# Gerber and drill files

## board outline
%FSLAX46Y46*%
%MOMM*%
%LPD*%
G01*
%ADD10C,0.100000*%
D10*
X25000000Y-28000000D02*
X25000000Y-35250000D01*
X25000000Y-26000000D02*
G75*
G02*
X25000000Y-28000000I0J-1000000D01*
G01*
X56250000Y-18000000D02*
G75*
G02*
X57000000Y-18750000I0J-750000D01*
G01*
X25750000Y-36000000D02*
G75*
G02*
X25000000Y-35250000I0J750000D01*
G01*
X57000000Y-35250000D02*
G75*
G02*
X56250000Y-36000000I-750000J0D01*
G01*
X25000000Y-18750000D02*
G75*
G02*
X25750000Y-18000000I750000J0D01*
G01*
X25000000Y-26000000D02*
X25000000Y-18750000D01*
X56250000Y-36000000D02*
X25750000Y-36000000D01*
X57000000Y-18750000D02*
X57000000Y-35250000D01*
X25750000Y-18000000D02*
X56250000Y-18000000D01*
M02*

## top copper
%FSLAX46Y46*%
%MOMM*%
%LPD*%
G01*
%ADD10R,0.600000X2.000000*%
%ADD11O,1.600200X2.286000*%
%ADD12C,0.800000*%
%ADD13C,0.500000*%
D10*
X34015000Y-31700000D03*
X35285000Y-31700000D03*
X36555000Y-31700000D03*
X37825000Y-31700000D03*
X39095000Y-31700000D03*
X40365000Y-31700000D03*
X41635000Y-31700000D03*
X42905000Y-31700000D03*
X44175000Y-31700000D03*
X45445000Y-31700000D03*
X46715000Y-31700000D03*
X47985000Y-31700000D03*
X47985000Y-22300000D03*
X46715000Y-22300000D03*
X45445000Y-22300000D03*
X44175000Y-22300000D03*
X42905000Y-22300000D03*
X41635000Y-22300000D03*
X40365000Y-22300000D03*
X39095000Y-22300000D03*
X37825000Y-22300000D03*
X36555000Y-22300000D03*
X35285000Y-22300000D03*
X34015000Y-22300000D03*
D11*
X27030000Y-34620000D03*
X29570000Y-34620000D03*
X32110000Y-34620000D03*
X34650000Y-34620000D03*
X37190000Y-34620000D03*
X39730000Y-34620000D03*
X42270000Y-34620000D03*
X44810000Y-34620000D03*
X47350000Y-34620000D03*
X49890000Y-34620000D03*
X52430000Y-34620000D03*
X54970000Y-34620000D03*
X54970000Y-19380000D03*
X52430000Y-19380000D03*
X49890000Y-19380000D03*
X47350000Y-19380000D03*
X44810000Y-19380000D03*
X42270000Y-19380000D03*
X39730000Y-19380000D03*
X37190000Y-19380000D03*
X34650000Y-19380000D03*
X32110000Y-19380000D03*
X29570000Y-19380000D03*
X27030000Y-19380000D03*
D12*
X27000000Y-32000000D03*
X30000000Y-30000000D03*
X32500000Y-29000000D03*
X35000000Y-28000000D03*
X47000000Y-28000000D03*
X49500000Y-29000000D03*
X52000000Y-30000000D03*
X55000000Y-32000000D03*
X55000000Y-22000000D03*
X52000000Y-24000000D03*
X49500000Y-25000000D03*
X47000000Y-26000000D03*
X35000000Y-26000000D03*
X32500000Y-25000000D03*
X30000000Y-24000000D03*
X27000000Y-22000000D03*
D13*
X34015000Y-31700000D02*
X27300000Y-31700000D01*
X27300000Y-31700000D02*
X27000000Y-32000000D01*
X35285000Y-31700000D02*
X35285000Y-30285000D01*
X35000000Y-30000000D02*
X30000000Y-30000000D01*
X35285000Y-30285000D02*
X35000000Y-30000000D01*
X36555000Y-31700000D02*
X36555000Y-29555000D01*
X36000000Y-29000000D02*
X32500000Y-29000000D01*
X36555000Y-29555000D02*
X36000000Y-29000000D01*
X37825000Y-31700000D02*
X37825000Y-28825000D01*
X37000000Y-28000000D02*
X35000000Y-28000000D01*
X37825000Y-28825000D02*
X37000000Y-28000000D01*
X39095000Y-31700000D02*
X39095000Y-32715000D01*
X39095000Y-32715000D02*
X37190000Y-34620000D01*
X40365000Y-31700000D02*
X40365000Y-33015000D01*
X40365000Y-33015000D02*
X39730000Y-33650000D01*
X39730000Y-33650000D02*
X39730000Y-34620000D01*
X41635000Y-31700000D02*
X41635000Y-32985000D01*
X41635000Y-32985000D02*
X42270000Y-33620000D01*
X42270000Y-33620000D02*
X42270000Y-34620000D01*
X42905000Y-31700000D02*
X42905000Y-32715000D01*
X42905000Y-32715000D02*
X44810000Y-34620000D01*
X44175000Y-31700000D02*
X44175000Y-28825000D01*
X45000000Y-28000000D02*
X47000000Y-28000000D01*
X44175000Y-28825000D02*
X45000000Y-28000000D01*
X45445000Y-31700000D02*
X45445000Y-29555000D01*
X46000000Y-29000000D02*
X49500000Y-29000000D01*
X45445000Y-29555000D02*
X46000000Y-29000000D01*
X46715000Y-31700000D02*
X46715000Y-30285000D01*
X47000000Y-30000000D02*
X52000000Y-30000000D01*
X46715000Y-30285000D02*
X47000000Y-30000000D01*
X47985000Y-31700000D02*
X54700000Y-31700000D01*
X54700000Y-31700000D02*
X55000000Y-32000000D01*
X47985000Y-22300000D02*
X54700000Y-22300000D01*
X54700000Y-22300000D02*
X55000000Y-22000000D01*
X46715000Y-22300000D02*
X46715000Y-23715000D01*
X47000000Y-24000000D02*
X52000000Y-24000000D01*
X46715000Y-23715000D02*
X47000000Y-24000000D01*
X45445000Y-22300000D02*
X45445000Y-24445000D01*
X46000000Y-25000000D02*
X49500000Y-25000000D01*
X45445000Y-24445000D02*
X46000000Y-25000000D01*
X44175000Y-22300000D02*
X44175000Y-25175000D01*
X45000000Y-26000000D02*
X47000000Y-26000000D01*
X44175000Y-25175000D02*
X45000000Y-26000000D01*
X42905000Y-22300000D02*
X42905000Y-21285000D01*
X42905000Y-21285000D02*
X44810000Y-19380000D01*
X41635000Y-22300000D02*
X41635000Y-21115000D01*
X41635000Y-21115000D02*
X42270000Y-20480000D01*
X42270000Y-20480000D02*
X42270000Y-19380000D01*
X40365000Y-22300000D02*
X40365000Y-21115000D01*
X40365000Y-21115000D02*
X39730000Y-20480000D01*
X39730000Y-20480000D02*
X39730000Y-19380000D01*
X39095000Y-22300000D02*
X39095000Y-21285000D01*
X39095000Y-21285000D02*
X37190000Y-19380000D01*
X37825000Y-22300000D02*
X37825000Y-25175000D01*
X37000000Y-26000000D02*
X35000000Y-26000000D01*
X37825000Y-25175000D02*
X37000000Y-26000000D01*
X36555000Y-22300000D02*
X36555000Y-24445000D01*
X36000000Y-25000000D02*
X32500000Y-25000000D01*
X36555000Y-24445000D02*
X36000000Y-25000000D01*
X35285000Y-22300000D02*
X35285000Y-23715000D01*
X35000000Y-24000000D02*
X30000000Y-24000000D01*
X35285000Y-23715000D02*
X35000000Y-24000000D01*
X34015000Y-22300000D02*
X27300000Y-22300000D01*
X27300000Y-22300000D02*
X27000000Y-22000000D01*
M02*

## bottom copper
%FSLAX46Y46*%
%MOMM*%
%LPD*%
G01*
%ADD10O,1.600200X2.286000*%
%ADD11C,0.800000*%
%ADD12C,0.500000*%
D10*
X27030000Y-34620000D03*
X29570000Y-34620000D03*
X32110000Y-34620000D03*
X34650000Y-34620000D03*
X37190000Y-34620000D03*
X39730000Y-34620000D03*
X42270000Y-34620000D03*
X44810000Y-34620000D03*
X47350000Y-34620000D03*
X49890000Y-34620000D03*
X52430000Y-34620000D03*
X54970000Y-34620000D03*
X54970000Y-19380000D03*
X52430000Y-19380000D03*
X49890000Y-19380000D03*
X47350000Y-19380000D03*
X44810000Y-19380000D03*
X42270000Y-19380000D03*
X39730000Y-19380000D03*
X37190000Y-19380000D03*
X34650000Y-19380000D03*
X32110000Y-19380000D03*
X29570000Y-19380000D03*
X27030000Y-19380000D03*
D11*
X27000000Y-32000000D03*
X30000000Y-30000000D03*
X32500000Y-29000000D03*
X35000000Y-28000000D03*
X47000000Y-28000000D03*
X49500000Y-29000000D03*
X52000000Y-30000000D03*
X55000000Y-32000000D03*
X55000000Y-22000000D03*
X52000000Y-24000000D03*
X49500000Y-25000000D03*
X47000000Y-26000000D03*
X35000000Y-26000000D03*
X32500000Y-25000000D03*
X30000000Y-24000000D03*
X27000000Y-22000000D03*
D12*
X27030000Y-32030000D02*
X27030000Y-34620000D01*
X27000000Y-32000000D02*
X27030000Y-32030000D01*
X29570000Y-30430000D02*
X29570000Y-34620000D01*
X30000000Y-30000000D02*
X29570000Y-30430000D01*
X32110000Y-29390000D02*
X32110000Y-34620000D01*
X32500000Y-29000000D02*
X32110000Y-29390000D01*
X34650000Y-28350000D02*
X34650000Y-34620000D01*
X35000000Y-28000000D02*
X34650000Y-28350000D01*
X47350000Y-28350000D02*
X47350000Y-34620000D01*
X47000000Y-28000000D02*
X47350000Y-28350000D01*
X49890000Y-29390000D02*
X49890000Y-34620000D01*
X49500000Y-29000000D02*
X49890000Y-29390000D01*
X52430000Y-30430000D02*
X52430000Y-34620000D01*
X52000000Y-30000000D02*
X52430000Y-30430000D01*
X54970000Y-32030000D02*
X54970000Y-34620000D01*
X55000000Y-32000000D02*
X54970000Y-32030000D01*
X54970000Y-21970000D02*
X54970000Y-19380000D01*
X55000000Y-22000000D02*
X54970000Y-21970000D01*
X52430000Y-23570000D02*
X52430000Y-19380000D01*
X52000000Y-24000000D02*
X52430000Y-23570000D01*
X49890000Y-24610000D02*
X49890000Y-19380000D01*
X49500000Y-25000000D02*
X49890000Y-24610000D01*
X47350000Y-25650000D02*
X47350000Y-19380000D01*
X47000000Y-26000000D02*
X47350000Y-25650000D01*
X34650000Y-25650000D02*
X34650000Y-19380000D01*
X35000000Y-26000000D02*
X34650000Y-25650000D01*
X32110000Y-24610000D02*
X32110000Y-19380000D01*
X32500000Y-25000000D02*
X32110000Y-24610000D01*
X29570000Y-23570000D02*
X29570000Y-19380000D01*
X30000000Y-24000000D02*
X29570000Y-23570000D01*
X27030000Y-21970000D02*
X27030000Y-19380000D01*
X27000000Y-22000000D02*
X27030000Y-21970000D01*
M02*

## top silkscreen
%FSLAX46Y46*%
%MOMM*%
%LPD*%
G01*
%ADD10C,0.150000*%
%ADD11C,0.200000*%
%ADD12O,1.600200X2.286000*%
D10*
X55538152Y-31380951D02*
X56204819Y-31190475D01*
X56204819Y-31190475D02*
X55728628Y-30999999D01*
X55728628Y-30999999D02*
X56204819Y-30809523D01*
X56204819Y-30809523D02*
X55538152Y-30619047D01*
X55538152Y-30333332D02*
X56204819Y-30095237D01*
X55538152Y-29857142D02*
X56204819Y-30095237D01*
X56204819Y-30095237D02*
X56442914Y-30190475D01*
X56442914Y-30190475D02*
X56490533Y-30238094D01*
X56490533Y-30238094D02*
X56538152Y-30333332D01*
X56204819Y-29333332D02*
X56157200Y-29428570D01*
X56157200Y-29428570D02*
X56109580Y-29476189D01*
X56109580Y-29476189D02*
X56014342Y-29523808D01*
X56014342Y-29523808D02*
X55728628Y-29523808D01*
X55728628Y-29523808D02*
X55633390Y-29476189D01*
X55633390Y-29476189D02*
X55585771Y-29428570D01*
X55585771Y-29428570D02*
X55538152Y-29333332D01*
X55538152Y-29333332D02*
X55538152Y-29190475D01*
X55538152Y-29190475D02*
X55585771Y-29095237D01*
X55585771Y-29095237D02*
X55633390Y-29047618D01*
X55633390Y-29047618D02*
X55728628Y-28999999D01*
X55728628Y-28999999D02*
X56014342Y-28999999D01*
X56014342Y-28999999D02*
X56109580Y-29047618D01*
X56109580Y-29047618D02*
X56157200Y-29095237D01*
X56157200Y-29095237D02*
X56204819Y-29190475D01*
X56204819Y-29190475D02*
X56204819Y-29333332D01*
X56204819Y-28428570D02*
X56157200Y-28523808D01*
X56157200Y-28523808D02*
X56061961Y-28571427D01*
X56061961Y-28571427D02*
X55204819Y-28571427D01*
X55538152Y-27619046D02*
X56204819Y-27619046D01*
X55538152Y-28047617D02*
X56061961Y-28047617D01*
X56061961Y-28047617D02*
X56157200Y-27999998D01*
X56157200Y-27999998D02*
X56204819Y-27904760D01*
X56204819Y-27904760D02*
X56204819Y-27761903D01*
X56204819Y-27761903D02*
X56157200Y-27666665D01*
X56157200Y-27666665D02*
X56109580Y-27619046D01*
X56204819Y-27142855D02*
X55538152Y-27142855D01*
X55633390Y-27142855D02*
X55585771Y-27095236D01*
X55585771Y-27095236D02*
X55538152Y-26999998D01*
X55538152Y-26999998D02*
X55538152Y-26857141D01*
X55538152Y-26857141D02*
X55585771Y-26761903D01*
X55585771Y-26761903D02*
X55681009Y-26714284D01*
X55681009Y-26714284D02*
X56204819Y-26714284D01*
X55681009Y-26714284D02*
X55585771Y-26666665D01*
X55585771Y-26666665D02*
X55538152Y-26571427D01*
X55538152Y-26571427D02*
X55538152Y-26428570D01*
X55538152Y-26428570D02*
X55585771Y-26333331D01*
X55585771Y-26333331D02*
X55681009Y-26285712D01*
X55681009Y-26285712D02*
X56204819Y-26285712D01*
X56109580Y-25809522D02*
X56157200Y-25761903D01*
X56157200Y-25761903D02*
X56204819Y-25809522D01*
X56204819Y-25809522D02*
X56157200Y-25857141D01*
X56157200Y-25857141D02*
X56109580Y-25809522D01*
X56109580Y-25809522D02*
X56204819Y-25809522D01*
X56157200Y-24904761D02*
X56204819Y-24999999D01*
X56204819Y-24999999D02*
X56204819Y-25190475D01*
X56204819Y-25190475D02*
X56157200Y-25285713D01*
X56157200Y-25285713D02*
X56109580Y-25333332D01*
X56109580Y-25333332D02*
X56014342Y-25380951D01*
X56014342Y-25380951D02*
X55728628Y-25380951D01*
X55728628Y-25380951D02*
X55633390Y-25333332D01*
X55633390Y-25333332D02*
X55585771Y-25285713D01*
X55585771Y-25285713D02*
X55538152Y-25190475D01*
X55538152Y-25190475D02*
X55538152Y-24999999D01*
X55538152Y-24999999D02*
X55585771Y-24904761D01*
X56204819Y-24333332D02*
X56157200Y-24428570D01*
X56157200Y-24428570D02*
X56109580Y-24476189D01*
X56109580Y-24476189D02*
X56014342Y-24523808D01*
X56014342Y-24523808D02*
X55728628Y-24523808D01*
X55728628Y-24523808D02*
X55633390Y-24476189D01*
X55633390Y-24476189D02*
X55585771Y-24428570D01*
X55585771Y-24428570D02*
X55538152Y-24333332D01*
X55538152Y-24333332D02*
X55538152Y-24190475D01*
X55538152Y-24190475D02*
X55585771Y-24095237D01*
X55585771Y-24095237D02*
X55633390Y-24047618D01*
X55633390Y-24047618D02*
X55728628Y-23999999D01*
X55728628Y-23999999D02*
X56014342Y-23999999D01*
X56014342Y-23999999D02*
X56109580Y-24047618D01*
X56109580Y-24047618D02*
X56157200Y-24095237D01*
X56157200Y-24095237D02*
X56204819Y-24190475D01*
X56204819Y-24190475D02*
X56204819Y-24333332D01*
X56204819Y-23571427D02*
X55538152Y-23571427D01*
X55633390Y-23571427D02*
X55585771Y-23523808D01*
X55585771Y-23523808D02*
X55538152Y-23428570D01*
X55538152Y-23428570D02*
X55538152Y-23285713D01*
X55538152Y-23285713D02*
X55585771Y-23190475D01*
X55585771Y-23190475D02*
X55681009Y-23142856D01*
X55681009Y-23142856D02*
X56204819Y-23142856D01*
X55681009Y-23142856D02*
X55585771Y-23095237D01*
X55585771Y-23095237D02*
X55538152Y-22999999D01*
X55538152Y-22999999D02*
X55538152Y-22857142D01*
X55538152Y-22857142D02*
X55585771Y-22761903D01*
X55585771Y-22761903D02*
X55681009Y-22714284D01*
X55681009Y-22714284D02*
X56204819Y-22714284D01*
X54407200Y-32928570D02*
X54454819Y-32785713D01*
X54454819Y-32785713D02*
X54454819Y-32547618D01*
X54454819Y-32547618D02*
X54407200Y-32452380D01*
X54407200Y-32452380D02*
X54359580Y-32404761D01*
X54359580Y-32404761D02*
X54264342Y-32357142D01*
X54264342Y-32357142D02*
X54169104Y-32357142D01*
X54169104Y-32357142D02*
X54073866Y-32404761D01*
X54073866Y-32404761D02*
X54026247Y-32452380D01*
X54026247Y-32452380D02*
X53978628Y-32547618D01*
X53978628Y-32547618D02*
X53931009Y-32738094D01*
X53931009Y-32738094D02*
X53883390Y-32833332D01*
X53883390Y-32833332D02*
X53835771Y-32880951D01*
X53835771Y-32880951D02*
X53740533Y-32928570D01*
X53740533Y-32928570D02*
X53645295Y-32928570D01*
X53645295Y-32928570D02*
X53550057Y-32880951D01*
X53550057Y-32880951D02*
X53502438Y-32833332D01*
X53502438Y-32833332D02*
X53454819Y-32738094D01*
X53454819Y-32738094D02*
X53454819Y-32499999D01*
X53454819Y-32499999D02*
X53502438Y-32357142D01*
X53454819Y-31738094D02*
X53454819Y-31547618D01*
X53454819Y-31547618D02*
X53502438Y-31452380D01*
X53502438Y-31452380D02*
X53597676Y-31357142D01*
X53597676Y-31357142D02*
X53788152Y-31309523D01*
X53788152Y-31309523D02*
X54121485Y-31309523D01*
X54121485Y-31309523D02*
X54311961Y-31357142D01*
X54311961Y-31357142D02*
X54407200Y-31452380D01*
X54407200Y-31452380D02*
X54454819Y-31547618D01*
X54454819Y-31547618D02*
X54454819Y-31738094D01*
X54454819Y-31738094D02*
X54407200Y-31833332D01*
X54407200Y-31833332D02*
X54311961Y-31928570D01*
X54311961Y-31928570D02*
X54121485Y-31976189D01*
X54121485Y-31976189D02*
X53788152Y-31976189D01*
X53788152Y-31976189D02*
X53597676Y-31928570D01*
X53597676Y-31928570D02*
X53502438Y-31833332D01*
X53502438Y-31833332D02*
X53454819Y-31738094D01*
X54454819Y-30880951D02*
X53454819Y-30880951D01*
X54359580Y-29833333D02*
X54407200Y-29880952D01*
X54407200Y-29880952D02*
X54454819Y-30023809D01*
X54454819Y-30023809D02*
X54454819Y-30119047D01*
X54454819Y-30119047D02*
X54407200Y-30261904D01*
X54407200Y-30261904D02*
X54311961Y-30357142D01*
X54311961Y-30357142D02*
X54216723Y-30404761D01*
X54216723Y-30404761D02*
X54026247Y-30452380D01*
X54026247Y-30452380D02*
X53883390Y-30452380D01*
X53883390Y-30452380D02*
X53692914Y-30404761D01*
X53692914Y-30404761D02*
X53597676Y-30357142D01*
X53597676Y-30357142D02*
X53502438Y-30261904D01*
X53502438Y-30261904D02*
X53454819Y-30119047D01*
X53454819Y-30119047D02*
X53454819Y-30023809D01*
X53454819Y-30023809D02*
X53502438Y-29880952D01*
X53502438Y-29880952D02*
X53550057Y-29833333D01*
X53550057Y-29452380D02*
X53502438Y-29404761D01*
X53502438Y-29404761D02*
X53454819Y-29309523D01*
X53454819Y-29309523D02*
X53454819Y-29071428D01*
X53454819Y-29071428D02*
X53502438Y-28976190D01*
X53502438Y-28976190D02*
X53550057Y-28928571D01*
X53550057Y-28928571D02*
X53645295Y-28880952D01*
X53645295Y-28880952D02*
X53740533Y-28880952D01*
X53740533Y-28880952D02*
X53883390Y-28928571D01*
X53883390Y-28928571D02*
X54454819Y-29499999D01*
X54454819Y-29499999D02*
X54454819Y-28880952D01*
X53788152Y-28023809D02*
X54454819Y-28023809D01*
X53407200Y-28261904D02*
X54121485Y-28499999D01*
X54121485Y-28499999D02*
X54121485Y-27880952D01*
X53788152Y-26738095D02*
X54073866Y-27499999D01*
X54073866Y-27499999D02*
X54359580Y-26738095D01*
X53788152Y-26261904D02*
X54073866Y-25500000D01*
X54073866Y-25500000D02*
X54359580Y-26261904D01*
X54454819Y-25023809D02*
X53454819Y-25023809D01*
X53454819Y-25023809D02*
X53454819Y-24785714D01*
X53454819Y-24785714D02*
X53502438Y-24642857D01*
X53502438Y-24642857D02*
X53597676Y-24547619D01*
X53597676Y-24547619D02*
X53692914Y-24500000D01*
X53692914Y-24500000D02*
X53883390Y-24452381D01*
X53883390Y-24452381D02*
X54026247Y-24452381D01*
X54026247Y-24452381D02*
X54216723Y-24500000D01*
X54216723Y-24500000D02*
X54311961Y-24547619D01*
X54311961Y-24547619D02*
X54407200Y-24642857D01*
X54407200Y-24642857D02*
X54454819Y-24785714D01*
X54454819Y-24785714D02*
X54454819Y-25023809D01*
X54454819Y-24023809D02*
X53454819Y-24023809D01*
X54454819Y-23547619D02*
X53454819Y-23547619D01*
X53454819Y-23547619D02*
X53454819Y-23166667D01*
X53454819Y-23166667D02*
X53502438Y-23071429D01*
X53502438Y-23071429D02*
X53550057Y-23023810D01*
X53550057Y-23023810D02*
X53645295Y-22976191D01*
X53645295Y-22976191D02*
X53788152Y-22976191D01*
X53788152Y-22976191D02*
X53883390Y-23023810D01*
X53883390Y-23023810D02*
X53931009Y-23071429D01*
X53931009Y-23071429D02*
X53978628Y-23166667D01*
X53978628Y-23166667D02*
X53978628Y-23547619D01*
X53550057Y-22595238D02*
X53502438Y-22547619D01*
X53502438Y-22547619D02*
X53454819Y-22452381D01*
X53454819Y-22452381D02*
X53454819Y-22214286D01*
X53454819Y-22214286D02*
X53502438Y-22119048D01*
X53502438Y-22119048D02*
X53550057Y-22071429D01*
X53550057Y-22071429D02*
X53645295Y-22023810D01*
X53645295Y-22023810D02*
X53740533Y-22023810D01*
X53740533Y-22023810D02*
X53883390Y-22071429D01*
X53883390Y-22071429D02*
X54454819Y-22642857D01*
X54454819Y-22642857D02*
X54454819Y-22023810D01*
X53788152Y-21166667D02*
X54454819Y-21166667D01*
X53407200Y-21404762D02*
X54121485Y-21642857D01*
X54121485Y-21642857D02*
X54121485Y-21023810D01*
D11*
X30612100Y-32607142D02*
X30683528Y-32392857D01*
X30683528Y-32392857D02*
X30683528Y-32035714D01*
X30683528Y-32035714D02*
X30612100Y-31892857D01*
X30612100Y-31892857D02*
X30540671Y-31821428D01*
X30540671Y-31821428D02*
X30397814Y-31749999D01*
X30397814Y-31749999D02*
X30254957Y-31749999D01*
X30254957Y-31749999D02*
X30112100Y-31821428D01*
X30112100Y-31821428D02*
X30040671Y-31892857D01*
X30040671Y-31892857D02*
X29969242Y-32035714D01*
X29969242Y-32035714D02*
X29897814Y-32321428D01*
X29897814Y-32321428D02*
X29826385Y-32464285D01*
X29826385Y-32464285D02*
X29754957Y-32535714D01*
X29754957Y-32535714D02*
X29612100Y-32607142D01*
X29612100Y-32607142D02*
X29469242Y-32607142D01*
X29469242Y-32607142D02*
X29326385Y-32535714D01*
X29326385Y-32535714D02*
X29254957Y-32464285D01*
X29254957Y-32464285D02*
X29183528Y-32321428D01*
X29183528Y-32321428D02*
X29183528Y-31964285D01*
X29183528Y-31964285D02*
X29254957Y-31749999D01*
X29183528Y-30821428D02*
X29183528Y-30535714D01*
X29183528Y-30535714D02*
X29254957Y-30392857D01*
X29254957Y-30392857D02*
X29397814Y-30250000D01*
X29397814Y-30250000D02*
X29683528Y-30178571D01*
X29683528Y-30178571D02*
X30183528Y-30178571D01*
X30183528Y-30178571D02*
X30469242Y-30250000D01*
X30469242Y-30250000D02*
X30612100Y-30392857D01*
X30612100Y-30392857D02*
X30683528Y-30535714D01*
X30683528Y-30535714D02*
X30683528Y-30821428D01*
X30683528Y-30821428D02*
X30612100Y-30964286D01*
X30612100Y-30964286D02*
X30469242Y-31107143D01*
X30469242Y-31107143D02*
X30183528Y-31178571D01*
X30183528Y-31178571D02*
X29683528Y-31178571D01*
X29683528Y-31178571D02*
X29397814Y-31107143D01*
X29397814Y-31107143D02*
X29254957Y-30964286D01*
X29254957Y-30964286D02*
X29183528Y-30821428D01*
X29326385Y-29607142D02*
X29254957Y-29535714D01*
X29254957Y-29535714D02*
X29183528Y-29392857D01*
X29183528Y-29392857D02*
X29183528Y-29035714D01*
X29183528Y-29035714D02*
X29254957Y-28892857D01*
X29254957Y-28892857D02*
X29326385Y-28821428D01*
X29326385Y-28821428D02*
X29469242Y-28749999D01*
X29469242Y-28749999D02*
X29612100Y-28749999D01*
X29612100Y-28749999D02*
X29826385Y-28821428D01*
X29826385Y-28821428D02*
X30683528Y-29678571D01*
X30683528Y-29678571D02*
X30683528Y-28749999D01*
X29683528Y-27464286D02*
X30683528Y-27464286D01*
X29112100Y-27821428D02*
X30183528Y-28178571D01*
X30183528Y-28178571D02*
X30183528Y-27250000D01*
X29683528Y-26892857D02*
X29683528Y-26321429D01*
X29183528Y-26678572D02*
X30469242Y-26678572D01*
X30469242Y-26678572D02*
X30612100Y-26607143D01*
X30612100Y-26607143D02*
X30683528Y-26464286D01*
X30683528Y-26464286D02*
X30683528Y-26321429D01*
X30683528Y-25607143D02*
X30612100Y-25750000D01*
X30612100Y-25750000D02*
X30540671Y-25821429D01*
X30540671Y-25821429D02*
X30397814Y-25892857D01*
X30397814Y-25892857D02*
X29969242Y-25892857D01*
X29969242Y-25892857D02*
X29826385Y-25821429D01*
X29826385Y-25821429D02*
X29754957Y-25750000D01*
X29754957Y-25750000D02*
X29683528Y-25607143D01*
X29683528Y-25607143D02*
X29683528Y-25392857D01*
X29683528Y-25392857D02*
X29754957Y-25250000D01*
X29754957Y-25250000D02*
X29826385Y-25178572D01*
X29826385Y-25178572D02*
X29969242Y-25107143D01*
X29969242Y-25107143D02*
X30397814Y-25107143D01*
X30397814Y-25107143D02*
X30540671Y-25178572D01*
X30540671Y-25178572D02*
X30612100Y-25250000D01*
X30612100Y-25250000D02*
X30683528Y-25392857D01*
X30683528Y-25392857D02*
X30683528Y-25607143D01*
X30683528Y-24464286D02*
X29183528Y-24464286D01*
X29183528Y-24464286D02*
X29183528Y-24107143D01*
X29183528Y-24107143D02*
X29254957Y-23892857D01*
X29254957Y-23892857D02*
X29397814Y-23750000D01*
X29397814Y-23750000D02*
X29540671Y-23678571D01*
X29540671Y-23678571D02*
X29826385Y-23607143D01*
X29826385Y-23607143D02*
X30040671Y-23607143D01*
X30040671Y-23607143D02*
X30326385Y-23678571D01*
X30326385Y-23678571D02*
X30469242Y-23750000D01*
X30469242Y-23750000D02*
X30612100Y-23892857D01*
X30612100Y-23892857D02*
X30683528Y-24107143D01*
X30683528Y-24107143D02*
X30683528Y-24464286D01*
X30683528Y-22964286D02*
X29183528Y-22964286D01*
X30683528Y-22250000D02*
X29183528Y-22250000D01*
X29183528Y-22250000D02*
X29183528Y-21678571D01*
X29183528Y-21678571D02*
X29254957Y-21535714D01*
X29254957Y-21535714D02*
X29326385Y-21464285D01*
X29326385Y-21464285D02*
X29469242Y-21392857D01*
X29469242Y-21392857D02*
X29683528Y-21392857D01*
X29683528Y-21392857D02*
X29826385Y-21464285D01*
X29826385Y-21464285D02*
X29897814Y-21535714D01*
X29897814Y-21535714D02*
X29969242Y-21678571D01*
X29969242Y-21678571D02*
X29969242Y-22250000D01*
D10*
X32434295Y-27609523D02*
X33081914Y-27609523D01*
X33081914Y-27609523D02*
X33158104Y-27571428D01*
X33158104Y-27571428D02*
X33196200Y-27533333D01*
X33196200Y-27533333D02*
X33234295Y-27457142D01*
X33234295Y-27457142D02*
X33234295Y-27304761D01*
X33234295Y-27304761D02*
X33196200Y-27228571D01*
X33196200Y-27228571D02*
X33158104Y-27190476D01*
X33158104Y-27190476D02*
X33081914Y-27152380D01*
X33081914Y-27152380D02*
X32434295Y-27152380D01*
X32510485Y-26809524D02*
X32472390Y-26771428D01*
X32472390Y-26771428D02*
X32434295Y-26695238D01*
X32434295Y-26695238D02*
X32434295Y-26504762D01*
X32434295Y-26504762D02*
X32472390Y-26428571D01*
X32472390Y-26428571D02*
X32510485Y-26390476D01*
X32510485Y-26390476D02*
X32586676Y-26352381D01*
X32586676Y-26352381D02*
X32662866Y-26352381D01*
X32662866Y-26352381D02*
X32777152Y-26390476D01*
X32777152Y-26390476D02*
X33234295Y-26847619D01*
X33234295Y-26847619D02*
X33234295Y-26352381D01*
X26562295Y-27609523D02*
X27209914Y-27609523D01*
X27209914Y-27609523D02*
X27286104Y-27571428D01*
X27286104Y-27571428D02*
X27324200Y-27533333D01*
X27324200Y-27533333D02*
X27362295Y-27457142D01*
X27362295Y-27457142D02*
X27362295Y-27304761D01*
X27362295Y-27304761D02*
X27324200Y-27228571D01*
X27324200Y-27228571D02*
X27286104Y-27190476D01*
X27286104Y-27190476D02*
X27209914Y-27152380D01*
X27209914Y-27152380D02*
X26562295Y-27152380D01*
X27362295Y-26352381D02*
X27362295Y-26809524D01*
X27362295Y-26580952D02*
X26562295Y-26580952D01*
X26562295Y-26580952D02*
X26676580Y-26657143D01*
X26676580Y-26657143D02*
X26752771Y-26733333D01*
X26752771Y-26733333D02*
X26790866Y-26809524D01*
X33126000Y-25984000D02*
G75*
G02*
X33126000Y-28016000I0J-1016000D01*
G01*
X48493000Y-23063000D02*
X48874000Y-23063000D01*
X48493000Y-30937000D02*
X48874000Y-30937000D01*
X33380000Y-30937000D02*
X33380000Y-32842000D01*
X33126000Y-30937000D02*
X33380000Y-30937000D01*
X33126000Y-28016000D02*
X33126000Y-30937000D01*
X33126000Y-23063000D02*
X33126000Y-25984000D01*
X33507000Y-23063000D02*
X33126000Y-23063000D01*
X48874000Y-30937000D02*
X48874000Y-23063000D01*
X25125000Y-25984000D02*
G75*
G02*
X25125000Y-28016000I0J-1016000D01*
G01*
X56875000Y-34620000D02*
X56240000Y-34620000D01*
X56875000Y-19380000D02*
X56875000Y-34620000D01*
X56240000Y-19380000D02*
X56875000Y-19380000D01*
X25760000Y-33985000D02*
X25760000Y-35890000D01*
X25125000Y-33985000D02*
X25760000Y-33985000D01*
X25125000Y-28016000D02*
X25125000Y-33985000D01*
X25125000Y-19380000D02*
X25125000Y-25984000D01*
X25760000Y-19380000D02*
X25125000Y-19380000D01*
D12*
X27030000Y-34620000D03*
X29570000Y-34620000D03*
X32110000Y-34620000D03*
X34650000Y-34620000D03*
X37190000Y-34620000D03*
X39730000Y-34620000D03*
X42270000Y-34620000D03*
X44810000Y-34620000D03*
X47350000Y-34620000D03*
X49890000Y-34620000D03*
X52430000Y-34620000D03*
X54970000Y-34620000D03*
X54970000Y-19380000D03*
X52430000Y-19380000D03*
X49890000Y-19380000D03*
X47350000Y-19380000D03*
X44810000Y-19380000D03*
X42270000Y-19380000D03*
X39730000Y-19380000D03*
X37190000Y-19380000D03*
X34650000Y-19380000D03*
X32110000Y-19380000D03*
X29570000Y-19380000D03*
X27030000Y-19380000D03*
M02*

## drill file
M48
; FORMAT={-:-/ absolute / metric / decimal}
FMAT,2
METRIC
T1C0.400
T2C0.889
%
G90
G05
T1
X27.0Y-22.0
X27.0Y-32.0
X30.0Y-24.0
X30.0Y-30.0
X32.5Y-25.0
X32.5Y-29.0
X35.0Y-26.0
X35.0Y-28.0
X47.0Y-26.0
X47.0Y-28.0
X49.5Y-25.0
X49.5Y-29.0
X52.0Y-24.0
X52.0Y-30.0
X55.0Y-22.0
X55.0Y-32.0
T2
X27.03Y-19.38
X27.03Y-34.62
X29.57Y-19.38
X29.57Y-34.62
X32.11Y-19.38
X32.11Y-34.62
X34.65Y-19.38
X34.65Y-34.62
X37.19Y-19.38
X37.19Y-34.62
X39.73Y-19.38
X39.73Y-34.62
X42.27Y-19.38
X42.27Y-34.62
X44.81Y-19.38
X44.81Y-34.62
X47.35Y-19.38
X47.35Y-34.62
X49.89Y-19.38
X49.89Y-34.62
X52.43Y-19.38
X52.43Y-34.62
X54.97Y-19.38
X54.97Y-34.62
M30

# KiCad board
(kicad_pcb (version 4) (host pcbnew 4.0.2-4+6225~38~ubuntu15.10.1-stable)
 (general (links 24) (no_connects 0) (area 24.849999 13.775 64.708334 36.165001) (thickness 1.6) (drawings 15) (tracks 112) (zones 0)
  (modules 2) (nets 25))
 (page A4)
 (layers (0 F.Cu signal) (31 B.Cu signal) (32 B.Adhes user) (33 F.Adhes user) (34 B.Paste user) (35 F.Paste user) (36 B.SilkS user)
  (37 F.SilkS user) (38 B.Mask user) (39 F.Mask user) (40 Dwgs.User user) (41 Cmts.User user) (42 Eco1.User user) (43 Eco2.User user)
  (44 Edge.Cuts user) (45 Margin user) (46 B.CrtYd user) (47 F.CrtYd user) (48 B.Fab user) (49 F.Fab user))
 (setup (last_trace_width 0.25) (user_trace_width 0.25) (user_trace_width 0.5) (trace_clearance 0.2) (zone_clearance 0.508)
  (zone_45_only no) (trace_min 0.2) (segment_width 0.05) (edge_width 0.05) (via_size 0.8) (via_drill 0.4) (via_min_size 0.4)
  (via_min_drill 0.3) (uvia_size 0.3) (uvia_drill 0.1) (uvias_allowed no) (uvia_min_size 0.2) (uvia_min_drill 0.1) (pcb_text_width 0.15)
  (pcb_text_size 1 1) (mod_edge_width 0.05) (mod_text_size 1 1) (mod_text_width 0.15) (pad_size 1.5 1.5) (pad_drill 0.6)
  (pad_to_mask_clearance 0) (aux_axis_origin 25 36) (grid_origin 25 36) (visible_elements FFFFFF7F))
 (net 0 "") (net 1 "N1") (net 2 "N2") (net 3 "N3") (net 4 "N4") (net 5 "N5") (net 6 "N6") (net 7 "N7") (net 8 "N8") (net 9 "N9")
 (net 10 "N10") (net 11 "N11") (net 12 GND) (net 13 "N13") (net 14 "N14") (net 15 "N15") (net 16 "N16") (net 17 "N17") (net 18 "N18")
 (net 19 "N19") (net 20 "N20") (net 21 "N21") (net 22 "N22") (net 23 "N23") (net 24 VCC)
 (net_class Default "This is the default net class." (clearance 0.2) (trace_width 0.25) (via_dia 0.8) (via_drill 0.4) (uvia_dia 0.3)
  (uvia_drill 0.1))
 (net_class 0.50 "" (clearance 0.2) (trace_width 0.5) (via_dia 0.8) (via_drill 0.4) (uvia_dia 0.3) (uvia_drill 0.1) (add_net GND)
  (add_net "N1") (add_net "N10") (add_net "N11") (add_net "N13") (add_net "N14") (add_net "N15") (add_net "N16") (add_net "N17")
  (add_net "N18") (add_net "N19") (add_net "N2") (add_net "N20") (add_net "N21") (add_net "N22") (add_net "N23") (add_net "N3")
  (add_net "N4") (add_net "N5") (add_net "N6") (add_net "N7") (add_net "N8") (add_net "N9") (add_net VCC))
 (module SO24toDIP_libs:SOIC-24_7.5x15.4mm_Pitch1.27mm (layer F.Cu) (at 41 27 90)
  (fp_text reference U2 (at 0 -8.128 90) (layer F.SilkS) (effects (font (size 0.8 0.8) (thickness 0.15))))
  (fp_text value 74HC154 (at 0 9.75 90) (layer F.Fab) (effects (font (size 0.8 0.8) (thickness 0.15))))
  (fp_arc (start 0 -7.874) (end 1.016 -7.874) (angle 180) (layer F.SilkS) (width 0.15))
  (fp_line (start 3.937 7.493) (end 3.937 7.874) (layer F.SilkS) (width 0.15))
  (fp_line (start -3.937 7.493) (end -3.937 7.874) (layer F.SilkS) (width 0.15))
  (fp_line (start -3.937 -7.62) (end -5.842 -7.62) (layer F.SilkS) (width 0.15))
  (fp_line (start -3.937 -7.874) (end -3.937 -7.62) (layer F.SilkS) (width 0.15))
  (fp_line (start -1.016 -7.874) (end -3.937 -7.874) (layer F.SilkS) (width 0.15))
  (fp_line (start 3.937 -7.874) (end 1.016 -7.874) (layer F.SilkS) (width 0.15))
  (fp_line (start 3.937 -7.493) (end 3.937 -7.874) (layer F.SilkS) (width 0.15))
  (fp_line (start -3.937 7.874) (end 3.937 7.874) (layer F.SilkS) (width 0.15))
  (pad 1 smd rect (at -4.7 -6.985 90) (size 2 0.6) (layers F.Cu F.Paste F.Mask) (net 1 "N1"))
  (pad 2 smd rect (at -4.7 -5.715 90) (size 2 0.6) (layers F.Cu F.Paste F.Mask) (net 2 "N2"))
  (pad 3 smd rect (at -4.7 -4.445 90) (size 2 0.6) (layers F.Cu F.Paste F.Mask) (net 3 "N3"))
  (pad 4 smd rect (at -4.7 -3.175 90) (size 2 0.6) (layers F.Cu F.Paste F.Mask) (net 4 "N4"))
  (pad 5 smd rect (at -4.7 -1.905 90) (size 2 0.6) (layers F.Cu F.Paste F.Mask) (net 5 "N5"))
  (pad 6 smd rect (at -4.7 -0.635 90) (size 2 0.6) (layers F.Cu F.Paste F.Mask) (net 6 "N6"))
  (pad 7 smd rect (at -4.7 0.635 90) (size 2 0.6) (layers F.Cu F.Paste F.Mask) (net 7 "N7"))
  (pad 8 smd rect (at -4.7 1.905 90) (size 2 0.6) (layers F.Cu F.Paste F.Mask) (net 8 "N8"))
  (pad 9 smd rect (at -4.7 3.175 90) (size 2 0.6) (layers F.Cu F.Paste F.Mask) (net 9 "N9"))
  (pad 10 smd rect (at -4.7 4.445 90) (size 2 0.6) (layers F.Cu F.Paste F.Mask) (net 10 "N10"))
  (pad 11 smd rect (at -4.7 5.715 90) (size 2 0.6) (layers F.Cu F.Paste F.Mask) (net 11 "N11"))
  (pad 12 smd rect (at -4.7 6.985 90) (size 2 0.6) (layers F.Cu F.Paste F.Mask) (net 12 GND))
  (pad 13 smd rect (at 4.7 6.985 90) (size 2 0.6) (layers F.Cu F.Paste F.Mask) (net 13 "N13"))
  (pad 14 smd rect (at 4.7 5.715 90) (size 2 0.6) (layers F.Cu F.Paste F.Mask) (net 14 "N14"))
  (pad 15 smd rect (at 4.7 4.445 90) (size 2 0.6) (layers F.Cu F.Paste F.Mask) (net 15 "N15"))
  (pad 16 smd rect (at 4.7 3.175 90) (size 2 0.6) (layers F.Cu F.Paste F.Mask) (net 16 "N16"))
  (pad 17 smd rect (at 4.7 1.905 90) (size 2 0.6) (layers F.Cu F.Paste F.Mask) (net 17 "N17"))
  (pad 18 smd rect (at 4.7 0.635 90) (size 2 0.6) (layers F.Cu F.Paste F.Mask) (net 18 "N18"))
  (pad 19 smd rect (at 4.7 -0.635 90) (size 2 0.6) (layers F.Cu F.Paste F.Mask) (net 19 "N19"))
  (pad 20 smd rect (at 4.7 -1.905 90) (size 2 0.6) (layers F.Cu F.Paste F.Mask) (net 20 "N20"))
  (pad 21 smd rect (at 4.7 -3.175 90) (size 2 0.6) (layers F.Cu F.Paste F.Mask) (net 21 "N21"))
  (pad 22 smd rect (at 4.7 -4.445 90) (size 2 0.6) (layers F.Cu F.Paste F.Mask) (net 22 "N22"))
  (pad 23 smd rect (at 4.7 -5.715 90) (size 2 0.6) (layers F.Cu F.Paste F.Mask) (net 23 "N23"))
  (pad 24 smd rect (at 4.7 -6.985 90) (size 2 0.6) (layers F.Cu F.Paste F.Mask) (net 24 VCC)))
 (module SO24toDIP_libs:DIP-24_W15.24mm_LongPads (layer F.Cu) (at 41 27)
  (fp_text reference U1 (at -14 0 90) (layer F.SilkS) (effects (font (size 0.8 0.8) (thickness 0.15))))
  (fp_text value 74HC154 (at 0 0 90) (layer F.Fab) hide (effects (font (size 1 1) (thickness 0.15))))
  (fp_arc (start -15.875 0) (end -15.875 -1.016) (angle 180) (layer F.SilkS) (width 0.15))
  (fp_line (start 15.875 7.62) (end 15.24 7.62) (layer F.SilkS) (width 0.15))
  (fp_line (start 15.875 -7.62) (end 15.875 7.62) (layer F.SilkS) (width 0.15))
  (fp_line (start 15.24 -7.62) (end 15.875 -7.62) (layer F.SilkS) (width 0.15))
  (fp_line (start -15.24 6.985) (end -15.24 8.89) (layer F.SilkS) (width 0.15))
  (fp_line (start -15.875 6.985) (end -15.24 6.985) (layer F.SilkS) (width 0.15))
  (fp_line (start -15.875 1.016) (end -15.875 6.985) (layer F.SilkS) (width 0.15))
  (fp_line (start -15.875 -7.62) (end -15.875 -1.016) (layer F.SilkS) (width 0.15))
  (fp_line (start -15.24 -7.62) (end -15.875 -7.62) (layer F.SilkS) (width 0.15))
  (pad 1 thru_hole oval (at -13.97 7.62 90) (size 2.286 1.6002) (drill 0.889) (layers *.Cu *.Mask F.SilkS) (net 1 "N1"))
  (pad 2 thru_hole oval (at -11.43 7.62 90) (size 2.286 1.6002) (drill 0.889) (layers *.Cu *.Mask F.SilkS) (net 2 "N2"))
  (pad 3 thru_hole oval (at -8.89 7.62 90) (size 2.286 1.6002) (drill 0.889) (layers *.Cu *.Mask F.SilkS) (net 3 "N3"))
  (pad 4 thru_hole oval (at -6.35 7.62 90) (size 2.286 1.6002) (drill 0.889) (layers *.Cu *.Mask F.SilkS) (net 4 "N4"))
  (pad 5 thru_hole oval (at -3.81 7.62 90) (size 2.286 1.6002) (drill 0.889) (layers *.Cu *.Mask F.SilkS) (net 5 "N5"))
  (pad 6 thru_hole oval (at -1.27 7.62 90) (size 2.286 1.6002) (drill 0.889) (layers *.Cu *.Mask F.SilkS) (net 6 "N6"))
  (pad 7 thru_hole oval (at 1.27 7.62 90) (size 2.286 1.6002) (drill 0.889) (layers *.Cu *.Mask F.SilkS) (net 7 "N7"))
  (pad 8 thru_hole oval (at 3.81 7.62 90) (size 2.286 1.6002) (drill 0.889) (layers *.Cu *.Mask F.SilkS) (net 8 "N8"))
  (pad 9 thru_hole oval (at 6.35 7.62 90) (size 2.286 1.6002) (drill 0.889) (layers *.Cu *.Mask F.SilkS) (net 9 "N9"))
  (pad 10 thru_hole oval (at 8.89 7.62 90) (size 2.286 1.6002) (drill 0.889) (layers *.Cu *.Mask F.SilkS) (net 10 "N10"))
  (pad 11 thru_hole oval (at 11.43 7.62 90) (size 2.286 1.6002) (drill 0.889) (layers *.Cu *.Mask F.SilkS) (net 11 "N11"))
  (pad 12 thru_hole oval (at 13.97 7.62 90) (size 2.286 1.6002) (drill 0.889) (layers *.Cu *.Mask F.SilkS) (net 12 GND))
  (pad 13 thru_hole oval (at 13.97 -7.62 90) (size 2.286 1.6002) (drill 0.889) (layers *.Cu *.Mask F.SilkS) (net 13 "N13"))
  (pad 14 thru_hole oval (at 11.43 -7.62 90) (size 2.286 1.6002) (drill 0.889) (layers *.Cu *.Mask F.SilkS) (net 14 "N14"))
  (pad 15 thru_hole oval (at 8.89 -7.62 90) (size 2.286 1.6002) (drill 0.889) (layers *.Cu *.Mask F.SilkS) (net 15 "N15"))
  (pad 16 thru_hole oval (at 6.35 -7.62 90) (size 2.286 1.6002) (drill 0.889) (layers *.Cu *.Mask F.SilkS) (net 16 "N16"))
  (pad 17 thru_hole oval (at 3.81 -7.62 90) (size 2.286 1.6002) (drill 0.889) (layers *.Cu *.Mask F.SilkS) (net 17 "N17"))
  (pad 18 thru_hole oval (at 1.27 -7.62 90) (size 2.286 1.6002) (drill 0.889) (layers *.Cu *.Mask F.SilkS) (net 18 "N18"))
  (pad 19 thru_hole oval (at -1.27 -7.62 90) (size 2.286 1.6002) (drill 0.889) (layers *.Cu *.Mask F.SilkS) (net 19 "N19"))
  (pad 20 thru_hole oval (at -3.81 -7.62 90) (size 2.286 1.6002) (drill 0.889) (layers *.Cu *.Mask F.SilkS) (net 20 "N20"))
  (pad 21 thru_hole oval (at -6.35 -7.62 90) (size 2.286 1.6002) (drill 0.889) (layers *.Cu *.Mask F.SilkS) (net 21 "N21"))
  (pad 22 thru_hole oval (at -8.89 -7.62 90) (size 2.286 1.6002) (drill 0.889) (layers *.Cu *.Mask F.SilkS) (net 22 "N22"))
  (pad 23 thru_hole oval (at -11.43 -7.62 90) (size 2.286 1.6002) (drill 0.889) (layers *.Cu *.Mask F.SilkS) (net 23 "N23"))
  (pad 24 thru_hole oval (at -13.97 -7.62 90) (size 2.286 1.6002) (drill 0.889) (layers *.Cu *.Mask F.SilkS) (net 24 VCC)))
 (gr_line (start 25 28) (end 25 35.25) (layer Edge.Cuts) (width 0.1))
 (gr_arc (start 25 27) (end 25 26) (angle 180) (layer Edge.Cuts) (width 0.1))
 (gr_arc (start 56.25 18.75) (end 56.25 18) (angle 90) (layer Edge.Cuts) (width 0.1))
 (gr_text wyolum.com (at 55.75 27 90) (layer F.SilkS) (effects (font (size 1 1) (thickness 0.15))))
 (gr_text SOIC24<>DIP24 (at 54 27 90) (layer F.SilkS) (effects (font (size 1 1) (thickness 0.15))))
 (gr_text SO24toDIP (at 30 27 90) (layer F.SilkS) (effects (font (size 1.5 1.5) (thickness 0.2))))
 (gr_arc (start 25.75 35.25) (end 25.75 36) (angle 90) (layer Edge.Cuts) (width 0.1))
 (gr_arc (start 56.25 35.25) (end 57 35.25) (angle 90) (layer Edge.Cuts) (width 0.1))
 (gr_arc (start 25.75 18.75) (end 25 18.75) (angle 90) (layer Edge.Cuts) (width 0.1))
 (gr_line (start 25 26) (end 25 18.75) (angle 90) (layer Edge.Cuts) (width 0.1))
 (gr_line (start 56.25 36) (end 25.75 36) (angle 90) (layer Edge.Cuts) (width 0.1))
 (gr_line (start 57 18.75) (end 57 35.25) (angle 90) (layer Edge.Cuts) (width 0.1))
 (gr_line (start 25.75 18) (end 56.25 18) (angle 90) (layer Edge.Cuts) (width 0.1))
 (segment (start 34.015 31.7) (end 27.3 31.7) (width 0.5) (layer F.Cu) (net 1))
 (segment (start 27.03 32.03) (end 27.03 34.62) (width 0.5) (layer B.Cu) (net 1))
 (segment (start 27 32) (end 27.03 32.03) (width 0.5) (layer B.Cu) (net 1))
 (via (at 27 32) (size 0.8) (drill 0.4) (layers F.Cu B.Cu) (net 1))
 (segment (start 27.3 31.7) (end 27 32) (width 0.5) (layer F.Cu) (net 1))
 (segment (start 35.285 31.7) (end 35.285 30.285) (width 0.5) (layer F.Cu) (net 2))
 (segment (start 29.57 30.43) (end 29.57 34.62) (width 0.5) (layer B.Cu) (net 2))
 (segment (start 30 30) (end 29.57 30.43) (width 0.5) (layer B.Cu) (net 2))
 (via (at 30 30) (size 0.8) (drill 0.4) (layers F.Cu B.Cu) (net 2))
 (segment (start 35 30) (end 30 30) (width 0.5) (layer F.Cu) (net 2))
 (segment (start 35.285 30.285) (end 35 30) (width 0.5) (layer F.Cu) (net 2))
 (segment (start 36.555 31.7) (end 36.555 29.555) (width 0.5) (layer F.Cu) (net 3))
 (segment (start 32.11 29.39) (end 32.11 34.62) (width 0.5) (layer B.Cu) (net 3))
 (segment (start 32.5 29) (end 32.11 29.39) (width 0.5) (layer B.Cu) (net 3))
 (via (at 32.5 29) (size 0.8) (drill 0.4) (layers F.Cu B.Cu) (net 3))
 (segment (start 36 29) (end 32.5 29) (width 0.5) (layer F.Cu) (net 3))
 (segment (start 36.555 29.555) (end 36 29) (width 0.5) (layer F.Cu) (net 3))
 (segment (start 37.825 31.7) (end 37.825 28.825) (width 0.5) (layer F.Cu) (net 4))
 (segment (start 34.65 28.35) (end 34.65 34.62) (width 0.5) (layer B.Cu) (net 4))
 (segment (start 35 28) (end 34.65 28.35) (width 0.5) (layer B.Cu) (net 4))
 (via (at 35 28) (size 0.8) (drill 0.4) (layers F.Cu B.Cu) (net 4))
 (segment (start 37 28) (end 35 28) (width 0.5) (layer F.Cu) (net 4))
 (segment (start 37.825 28.825) (end 37 28) (width 0.5) (layer F.Cu) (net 4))
 (segment (start 39.095 31.7) (end 39.095 32.715) (width 0.5) (layer F.Cu) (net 5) (status 10))
 (segment (start 39.095 32.715) (end 37.19 34.62) (width 0.5) (layer F.Cu) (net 5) (status 20))
 (segment (start 40.365 31.7) (end 40.365 33.015) (width 0.5) (layer F.Cu) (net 6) (status 10))
 (segment (start 40.365 33.015) (end 39.73 33.65) (width 0.5) (layer F.Cu) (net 6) (status 20))
 (segment (start 39.73 33.65) (end 39.73 34.62) (width 0.5) (layer F.Cu) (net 6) (status 30))
 (segment (start 41.635 31.7) (end 41.635 32.985) (width 0.5) (layer F.Cu) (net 7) (status 30))
 (segment (start 41.635 32.985) (end 42.27 33.62) (width 0.5) (layer F.Cu) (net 7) (status 10))
 (segment (start 42.27 33.62) (end 42.27 34.62) (width 0.5) (layer F.Cu) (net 7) (status 20))
 (segment (start 42.905 31.7) (end 42.905 32.715) (width 0.5) (layer F.Cu) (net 8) (status 10))
 (segment (start 42.905 32.715) (end 44.81 34.62) (width 0.5) (layer F.Cu) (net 8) (status 20))
 (segment (start 44.175 31.7) (end 44.175 28.825) (width 0.5) (layer F.Cu) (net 9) (status 10))
 (segment (start 47.35 28.35) (end 47.35 34.62) (width 0.5) (layer B.Cu) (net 9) (status 20))
 (segment (start 47 28) (end 47.35 28.35) (width 0.5) (layer B.Cu) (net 9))
 (via (at 47 28) (size 0.8) (drill 0.4) (layers F.Cu B.Cu) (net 9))
 (segment (start 45 28) (end 47 28) (width 0.5) (layer F.Cu) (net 9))
 (segment (start 44.175 28.825) (end 45 28) (width 0.5) (layer F.Cu) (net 9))
 (segment (start 45.445 31.7) (end 45.445 29.555) (width 0.5) (layer F.Cu) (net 10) (status 10))
 (segment (start 49.89 29.39) (end 49.89 34.62) (width 0.5) (layer B.Cu) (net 10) (status 20))
 (segment (start 49.5 29) (end 49.89 29.39) (width 0.5) (layer B.Cu) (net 10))
 (via (at 49.5 29) (size 0.8) (drill 0.4) (layers F.Cu B.Cu) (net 10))
 (segment (start 46 29) (end 49.5 29) (width 0.5) (layer F.Cu) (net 10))
 (segment (start 45.445 29.555) (end 46 29) (width 0.5) (layer F.Cu) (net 10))
 (segment (start 46.715 31.7) (end 46.715 30.285) (width 0.5) (layer F.Cu) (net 11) (status 10))
 (segment (start 52.43 30.43) (end 52.43 34.62) (width 0.5) (layer B.Cu) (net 11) (status 20))
 (segment (start 52 30) (end 52.43 30.43) (width 0.5) (layer B.Cu) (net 11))
 (via (at 52 30) (size 0.8) (drill 0.4) (layers F.Cu B.Cu) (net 11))
 (segment (start 47 30) (end 52 30) (width 0.5) (layer F.Cu) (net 11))
 (segment (start 46.715 30.285) (end 47 30) (width 0.5) (layer F.Cu) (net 11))
 (segment (start 47.985 31.7) (end 54.7 31.7) (width 0.5) (layer F.Cu) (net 12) (status 10))
 (segment (start 54.97 32.03) (end 54.97 34.62) (width 0.5) (layer B.Cu) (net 12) (status 20))
 (segment (start 55 32) (end 54.97 32.03) (width 0.5) (layer B.Cu) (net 12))
 (via (at 55 32) (size 0.8) (drill 0.4) (layers F.Cu B.Cu) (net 12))
 (segment (start 54.7 31.7) (end 55 32) (width 0.5) (layer F.Cu) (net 12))
 (segment (start 47.985 22.3) (end 54.7 22.3) (width 0.5) (layer F.Cu) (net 13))
 (segment (start 54.97 21.97) (end 54.97 19.38) (width 0.5) (layer B.Cu) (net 13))
 (segment (start 55 22) (end 54.97 21.97) (width 0.5) (layer B.Cu) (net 13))
 (via (at 55 22) (size 0.8) (drill 0.4) (layers F.Cu B.Cu) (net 13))
 (segment (start 54.7 22.3) (end 55 22) (width 0.5) (layer F.Cu) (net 13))
 (segment (start 46.715 22.3) (end 46.715 23.715) (width 0.5) (layer F.Cu) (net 14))
 (segment (start 52.43 23.57) (end 52.43 19.38) (width 0.5) (layer B.Cu) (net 14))
 (segment (start 52 24) (end 52.43 23.57) (width 0.5) (layer B.Cu) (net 14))
 (via (at 52 24) (size 0.8) (drill 0.4) (layers F.Cu B.Cu) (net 14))
 (segment (start 47 24) (end 52 24) (width 0.5) (layer F.Cu) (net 14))
 (segment (start 46.715 23.715) (end 47 24) (width 0.5) (layer F.Cu) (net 14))
 (segment (start 45.445 22.3) (end 45.445 24.445) (width 0.5) (layer F.Cu) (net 15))
 (segment (start 49.89 24.61) (end 49.89 19.38) (width 0.5) (layer B.Cu) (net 15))
 (segment (start 49.5 25) (end 49.89 24.61) (width 0.5) (layer B.Cu) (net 15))
 (via (at 49.5 25) (size 0.8) (drill 0.4) (layers F.Cu B.Cu) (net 15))
 (segment (start 46 25) (end 49.5 25) (width 0.5) (layer F.Cu) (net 15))
 (segment (start 45.445 24.445) (end 46 25) (width 0.5) (layer F.Cu) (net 15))
 (segment (start 44.175 22.3) (end 44.175 25.175) (width 0.5) (layer F.Cu) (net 16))
 (segment (start 47.35 25.65) (end 47.35 19.38) (width 0.5) (layer B.Cu) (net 16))
 (segment (start 47 26) (end 47.35 25.65) (width 0.5) (layer B.Cu) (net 16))
 (via (at 47 26) (size 0.8) (drill 0.4) (layers F.Cu B.Cu) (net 16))
 (segment (start 45 26) (end 47 26) (width 0.5) (layer F.Cu) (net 16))
 (segment (start 44.175 25.175) (end 45 26) (width 0.5) (layer F.Cu) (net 16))
 (segment (start 42.905 22.3) (end 42.905 21.285) (width 0.5) (layer F.Cu) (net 17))
 (segment (start 42.905 21.285) (end 44.81 19.38) (width 0.5) (layer F.Cu) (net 17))
 (segment (start 41.635 22.3) (end 41.635 21.115) (width 0.5) (layer F.Cu) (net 18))
 (segment (start 41.635 21.115) (end 42.27 20.48) (width 0.5) (layer F.Cu) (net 18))
 (segment (start 42.27 20.48) (end 42.27 19.38) (width 0.5) (layer F.Cu) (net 18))
 (segment (start 40.365 22.3) (end 40.365 21.115) (width 0.5) (layer F.Cu) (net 19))
 (segment (start 40.365 21.115) (end 39.73 20.48) (width 0.5) (layer F.Cu) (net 19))
 (segment (start 39.73 20.48) (end 39.73 19.38) (width 0.5) (layer F.Cu) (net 19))
 (segment (start 39.095 22.3) (end 39.095 21.285) (width 0.5) (layer F.Cu) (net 20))
 (segment (start 39.095 21.285) (end 37.19 19.38) (width 0.5) (layer F.Cu) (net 20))
 (segment (start 37.825 22.3) (end 37.825 25.175) (width 0.5) (layer F.Cu) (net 21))
 (segment (start 34.65 25.65) (end 34.65 19.38) (width 0.5) (layer B.Cu) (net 21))
 (segment (start 35 26) (end 34.65 25.65) (width 0.5) (layer B.Cu) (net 21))
 (via (at 35 26) (size 0.8) (drill 0.4) (layers F.Cu B.Cu) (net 21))
 (segment (start 37 26) (end 35 26) (width 0.5) (layer F.Cu) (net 21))
 (segment (start 37.825 25.175) (end 37 26) (width 0.5) (layer F.Cu) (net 21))
 (segment (start 36.555 22.3) (end 36.555 24.445) (width 0.5) (layer F.Cu) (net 22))
 (segment (start 32.11 24.61) (end 32.11 19.38) (width 0.5) (layer B.Cu) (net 22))
 (segment (start 32.5 25) (end 32.11 24.61) (width 0.5) (layer B.Cu) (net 22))
 (via (at 32.5 25) (size 0.8) (drill 0.4) (layers F.Cu B.Cu) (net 22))
 (segment (start 36 25) (end 32.5 25) (width 0.5) (layer F.Cu) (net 22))
 (segment (start 36.555 24.445) (end 36 25) (width 0.5) (layer F.Cu) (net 22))
 (segment (start 35.285 22.3) (end 35.285 23.715) (width 0.5) (layer F.Cu) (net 23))
 (segment (start 29.57 23.57) (end 29.57 19.38) (width 0.5) (layer B.Cu) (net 23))
 (segment (start 30 24) (end 29.57 23.57) (width 0.5) (layer B.Cu) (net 23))
 (via (at 30 24) (size 0.8) (drill 0.4) (layers F.Cu B.Cu) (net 23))
 (segment (start 35 24) (end 30 24) (width 0.5) (layer F.Cu) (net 23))
 (segment (start 35.285 23.715) (end 35 24) (width 0.5) (layer F.Cu) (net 23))
 (segment (start 34.015 22.3) (end 27.3 22.3) (width 0.5) (layer F.Cu) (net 24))
 (segment (start 27.03 21.97) (end 27.03 19.38) (width 0.5) (layer B.Cu) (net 24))
 (segment (start 27 22) (end 27.03 21.97) (width 0.5) (layer B.Cu) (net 24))
 (via (at 27 22) (size 0.8) (drill 0.4) (layers F.Cu B.Cu) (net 24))
 (segment (start 27.3 22.3) (end 27 22) (width 0.5) (layer F.Cu) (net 24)))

